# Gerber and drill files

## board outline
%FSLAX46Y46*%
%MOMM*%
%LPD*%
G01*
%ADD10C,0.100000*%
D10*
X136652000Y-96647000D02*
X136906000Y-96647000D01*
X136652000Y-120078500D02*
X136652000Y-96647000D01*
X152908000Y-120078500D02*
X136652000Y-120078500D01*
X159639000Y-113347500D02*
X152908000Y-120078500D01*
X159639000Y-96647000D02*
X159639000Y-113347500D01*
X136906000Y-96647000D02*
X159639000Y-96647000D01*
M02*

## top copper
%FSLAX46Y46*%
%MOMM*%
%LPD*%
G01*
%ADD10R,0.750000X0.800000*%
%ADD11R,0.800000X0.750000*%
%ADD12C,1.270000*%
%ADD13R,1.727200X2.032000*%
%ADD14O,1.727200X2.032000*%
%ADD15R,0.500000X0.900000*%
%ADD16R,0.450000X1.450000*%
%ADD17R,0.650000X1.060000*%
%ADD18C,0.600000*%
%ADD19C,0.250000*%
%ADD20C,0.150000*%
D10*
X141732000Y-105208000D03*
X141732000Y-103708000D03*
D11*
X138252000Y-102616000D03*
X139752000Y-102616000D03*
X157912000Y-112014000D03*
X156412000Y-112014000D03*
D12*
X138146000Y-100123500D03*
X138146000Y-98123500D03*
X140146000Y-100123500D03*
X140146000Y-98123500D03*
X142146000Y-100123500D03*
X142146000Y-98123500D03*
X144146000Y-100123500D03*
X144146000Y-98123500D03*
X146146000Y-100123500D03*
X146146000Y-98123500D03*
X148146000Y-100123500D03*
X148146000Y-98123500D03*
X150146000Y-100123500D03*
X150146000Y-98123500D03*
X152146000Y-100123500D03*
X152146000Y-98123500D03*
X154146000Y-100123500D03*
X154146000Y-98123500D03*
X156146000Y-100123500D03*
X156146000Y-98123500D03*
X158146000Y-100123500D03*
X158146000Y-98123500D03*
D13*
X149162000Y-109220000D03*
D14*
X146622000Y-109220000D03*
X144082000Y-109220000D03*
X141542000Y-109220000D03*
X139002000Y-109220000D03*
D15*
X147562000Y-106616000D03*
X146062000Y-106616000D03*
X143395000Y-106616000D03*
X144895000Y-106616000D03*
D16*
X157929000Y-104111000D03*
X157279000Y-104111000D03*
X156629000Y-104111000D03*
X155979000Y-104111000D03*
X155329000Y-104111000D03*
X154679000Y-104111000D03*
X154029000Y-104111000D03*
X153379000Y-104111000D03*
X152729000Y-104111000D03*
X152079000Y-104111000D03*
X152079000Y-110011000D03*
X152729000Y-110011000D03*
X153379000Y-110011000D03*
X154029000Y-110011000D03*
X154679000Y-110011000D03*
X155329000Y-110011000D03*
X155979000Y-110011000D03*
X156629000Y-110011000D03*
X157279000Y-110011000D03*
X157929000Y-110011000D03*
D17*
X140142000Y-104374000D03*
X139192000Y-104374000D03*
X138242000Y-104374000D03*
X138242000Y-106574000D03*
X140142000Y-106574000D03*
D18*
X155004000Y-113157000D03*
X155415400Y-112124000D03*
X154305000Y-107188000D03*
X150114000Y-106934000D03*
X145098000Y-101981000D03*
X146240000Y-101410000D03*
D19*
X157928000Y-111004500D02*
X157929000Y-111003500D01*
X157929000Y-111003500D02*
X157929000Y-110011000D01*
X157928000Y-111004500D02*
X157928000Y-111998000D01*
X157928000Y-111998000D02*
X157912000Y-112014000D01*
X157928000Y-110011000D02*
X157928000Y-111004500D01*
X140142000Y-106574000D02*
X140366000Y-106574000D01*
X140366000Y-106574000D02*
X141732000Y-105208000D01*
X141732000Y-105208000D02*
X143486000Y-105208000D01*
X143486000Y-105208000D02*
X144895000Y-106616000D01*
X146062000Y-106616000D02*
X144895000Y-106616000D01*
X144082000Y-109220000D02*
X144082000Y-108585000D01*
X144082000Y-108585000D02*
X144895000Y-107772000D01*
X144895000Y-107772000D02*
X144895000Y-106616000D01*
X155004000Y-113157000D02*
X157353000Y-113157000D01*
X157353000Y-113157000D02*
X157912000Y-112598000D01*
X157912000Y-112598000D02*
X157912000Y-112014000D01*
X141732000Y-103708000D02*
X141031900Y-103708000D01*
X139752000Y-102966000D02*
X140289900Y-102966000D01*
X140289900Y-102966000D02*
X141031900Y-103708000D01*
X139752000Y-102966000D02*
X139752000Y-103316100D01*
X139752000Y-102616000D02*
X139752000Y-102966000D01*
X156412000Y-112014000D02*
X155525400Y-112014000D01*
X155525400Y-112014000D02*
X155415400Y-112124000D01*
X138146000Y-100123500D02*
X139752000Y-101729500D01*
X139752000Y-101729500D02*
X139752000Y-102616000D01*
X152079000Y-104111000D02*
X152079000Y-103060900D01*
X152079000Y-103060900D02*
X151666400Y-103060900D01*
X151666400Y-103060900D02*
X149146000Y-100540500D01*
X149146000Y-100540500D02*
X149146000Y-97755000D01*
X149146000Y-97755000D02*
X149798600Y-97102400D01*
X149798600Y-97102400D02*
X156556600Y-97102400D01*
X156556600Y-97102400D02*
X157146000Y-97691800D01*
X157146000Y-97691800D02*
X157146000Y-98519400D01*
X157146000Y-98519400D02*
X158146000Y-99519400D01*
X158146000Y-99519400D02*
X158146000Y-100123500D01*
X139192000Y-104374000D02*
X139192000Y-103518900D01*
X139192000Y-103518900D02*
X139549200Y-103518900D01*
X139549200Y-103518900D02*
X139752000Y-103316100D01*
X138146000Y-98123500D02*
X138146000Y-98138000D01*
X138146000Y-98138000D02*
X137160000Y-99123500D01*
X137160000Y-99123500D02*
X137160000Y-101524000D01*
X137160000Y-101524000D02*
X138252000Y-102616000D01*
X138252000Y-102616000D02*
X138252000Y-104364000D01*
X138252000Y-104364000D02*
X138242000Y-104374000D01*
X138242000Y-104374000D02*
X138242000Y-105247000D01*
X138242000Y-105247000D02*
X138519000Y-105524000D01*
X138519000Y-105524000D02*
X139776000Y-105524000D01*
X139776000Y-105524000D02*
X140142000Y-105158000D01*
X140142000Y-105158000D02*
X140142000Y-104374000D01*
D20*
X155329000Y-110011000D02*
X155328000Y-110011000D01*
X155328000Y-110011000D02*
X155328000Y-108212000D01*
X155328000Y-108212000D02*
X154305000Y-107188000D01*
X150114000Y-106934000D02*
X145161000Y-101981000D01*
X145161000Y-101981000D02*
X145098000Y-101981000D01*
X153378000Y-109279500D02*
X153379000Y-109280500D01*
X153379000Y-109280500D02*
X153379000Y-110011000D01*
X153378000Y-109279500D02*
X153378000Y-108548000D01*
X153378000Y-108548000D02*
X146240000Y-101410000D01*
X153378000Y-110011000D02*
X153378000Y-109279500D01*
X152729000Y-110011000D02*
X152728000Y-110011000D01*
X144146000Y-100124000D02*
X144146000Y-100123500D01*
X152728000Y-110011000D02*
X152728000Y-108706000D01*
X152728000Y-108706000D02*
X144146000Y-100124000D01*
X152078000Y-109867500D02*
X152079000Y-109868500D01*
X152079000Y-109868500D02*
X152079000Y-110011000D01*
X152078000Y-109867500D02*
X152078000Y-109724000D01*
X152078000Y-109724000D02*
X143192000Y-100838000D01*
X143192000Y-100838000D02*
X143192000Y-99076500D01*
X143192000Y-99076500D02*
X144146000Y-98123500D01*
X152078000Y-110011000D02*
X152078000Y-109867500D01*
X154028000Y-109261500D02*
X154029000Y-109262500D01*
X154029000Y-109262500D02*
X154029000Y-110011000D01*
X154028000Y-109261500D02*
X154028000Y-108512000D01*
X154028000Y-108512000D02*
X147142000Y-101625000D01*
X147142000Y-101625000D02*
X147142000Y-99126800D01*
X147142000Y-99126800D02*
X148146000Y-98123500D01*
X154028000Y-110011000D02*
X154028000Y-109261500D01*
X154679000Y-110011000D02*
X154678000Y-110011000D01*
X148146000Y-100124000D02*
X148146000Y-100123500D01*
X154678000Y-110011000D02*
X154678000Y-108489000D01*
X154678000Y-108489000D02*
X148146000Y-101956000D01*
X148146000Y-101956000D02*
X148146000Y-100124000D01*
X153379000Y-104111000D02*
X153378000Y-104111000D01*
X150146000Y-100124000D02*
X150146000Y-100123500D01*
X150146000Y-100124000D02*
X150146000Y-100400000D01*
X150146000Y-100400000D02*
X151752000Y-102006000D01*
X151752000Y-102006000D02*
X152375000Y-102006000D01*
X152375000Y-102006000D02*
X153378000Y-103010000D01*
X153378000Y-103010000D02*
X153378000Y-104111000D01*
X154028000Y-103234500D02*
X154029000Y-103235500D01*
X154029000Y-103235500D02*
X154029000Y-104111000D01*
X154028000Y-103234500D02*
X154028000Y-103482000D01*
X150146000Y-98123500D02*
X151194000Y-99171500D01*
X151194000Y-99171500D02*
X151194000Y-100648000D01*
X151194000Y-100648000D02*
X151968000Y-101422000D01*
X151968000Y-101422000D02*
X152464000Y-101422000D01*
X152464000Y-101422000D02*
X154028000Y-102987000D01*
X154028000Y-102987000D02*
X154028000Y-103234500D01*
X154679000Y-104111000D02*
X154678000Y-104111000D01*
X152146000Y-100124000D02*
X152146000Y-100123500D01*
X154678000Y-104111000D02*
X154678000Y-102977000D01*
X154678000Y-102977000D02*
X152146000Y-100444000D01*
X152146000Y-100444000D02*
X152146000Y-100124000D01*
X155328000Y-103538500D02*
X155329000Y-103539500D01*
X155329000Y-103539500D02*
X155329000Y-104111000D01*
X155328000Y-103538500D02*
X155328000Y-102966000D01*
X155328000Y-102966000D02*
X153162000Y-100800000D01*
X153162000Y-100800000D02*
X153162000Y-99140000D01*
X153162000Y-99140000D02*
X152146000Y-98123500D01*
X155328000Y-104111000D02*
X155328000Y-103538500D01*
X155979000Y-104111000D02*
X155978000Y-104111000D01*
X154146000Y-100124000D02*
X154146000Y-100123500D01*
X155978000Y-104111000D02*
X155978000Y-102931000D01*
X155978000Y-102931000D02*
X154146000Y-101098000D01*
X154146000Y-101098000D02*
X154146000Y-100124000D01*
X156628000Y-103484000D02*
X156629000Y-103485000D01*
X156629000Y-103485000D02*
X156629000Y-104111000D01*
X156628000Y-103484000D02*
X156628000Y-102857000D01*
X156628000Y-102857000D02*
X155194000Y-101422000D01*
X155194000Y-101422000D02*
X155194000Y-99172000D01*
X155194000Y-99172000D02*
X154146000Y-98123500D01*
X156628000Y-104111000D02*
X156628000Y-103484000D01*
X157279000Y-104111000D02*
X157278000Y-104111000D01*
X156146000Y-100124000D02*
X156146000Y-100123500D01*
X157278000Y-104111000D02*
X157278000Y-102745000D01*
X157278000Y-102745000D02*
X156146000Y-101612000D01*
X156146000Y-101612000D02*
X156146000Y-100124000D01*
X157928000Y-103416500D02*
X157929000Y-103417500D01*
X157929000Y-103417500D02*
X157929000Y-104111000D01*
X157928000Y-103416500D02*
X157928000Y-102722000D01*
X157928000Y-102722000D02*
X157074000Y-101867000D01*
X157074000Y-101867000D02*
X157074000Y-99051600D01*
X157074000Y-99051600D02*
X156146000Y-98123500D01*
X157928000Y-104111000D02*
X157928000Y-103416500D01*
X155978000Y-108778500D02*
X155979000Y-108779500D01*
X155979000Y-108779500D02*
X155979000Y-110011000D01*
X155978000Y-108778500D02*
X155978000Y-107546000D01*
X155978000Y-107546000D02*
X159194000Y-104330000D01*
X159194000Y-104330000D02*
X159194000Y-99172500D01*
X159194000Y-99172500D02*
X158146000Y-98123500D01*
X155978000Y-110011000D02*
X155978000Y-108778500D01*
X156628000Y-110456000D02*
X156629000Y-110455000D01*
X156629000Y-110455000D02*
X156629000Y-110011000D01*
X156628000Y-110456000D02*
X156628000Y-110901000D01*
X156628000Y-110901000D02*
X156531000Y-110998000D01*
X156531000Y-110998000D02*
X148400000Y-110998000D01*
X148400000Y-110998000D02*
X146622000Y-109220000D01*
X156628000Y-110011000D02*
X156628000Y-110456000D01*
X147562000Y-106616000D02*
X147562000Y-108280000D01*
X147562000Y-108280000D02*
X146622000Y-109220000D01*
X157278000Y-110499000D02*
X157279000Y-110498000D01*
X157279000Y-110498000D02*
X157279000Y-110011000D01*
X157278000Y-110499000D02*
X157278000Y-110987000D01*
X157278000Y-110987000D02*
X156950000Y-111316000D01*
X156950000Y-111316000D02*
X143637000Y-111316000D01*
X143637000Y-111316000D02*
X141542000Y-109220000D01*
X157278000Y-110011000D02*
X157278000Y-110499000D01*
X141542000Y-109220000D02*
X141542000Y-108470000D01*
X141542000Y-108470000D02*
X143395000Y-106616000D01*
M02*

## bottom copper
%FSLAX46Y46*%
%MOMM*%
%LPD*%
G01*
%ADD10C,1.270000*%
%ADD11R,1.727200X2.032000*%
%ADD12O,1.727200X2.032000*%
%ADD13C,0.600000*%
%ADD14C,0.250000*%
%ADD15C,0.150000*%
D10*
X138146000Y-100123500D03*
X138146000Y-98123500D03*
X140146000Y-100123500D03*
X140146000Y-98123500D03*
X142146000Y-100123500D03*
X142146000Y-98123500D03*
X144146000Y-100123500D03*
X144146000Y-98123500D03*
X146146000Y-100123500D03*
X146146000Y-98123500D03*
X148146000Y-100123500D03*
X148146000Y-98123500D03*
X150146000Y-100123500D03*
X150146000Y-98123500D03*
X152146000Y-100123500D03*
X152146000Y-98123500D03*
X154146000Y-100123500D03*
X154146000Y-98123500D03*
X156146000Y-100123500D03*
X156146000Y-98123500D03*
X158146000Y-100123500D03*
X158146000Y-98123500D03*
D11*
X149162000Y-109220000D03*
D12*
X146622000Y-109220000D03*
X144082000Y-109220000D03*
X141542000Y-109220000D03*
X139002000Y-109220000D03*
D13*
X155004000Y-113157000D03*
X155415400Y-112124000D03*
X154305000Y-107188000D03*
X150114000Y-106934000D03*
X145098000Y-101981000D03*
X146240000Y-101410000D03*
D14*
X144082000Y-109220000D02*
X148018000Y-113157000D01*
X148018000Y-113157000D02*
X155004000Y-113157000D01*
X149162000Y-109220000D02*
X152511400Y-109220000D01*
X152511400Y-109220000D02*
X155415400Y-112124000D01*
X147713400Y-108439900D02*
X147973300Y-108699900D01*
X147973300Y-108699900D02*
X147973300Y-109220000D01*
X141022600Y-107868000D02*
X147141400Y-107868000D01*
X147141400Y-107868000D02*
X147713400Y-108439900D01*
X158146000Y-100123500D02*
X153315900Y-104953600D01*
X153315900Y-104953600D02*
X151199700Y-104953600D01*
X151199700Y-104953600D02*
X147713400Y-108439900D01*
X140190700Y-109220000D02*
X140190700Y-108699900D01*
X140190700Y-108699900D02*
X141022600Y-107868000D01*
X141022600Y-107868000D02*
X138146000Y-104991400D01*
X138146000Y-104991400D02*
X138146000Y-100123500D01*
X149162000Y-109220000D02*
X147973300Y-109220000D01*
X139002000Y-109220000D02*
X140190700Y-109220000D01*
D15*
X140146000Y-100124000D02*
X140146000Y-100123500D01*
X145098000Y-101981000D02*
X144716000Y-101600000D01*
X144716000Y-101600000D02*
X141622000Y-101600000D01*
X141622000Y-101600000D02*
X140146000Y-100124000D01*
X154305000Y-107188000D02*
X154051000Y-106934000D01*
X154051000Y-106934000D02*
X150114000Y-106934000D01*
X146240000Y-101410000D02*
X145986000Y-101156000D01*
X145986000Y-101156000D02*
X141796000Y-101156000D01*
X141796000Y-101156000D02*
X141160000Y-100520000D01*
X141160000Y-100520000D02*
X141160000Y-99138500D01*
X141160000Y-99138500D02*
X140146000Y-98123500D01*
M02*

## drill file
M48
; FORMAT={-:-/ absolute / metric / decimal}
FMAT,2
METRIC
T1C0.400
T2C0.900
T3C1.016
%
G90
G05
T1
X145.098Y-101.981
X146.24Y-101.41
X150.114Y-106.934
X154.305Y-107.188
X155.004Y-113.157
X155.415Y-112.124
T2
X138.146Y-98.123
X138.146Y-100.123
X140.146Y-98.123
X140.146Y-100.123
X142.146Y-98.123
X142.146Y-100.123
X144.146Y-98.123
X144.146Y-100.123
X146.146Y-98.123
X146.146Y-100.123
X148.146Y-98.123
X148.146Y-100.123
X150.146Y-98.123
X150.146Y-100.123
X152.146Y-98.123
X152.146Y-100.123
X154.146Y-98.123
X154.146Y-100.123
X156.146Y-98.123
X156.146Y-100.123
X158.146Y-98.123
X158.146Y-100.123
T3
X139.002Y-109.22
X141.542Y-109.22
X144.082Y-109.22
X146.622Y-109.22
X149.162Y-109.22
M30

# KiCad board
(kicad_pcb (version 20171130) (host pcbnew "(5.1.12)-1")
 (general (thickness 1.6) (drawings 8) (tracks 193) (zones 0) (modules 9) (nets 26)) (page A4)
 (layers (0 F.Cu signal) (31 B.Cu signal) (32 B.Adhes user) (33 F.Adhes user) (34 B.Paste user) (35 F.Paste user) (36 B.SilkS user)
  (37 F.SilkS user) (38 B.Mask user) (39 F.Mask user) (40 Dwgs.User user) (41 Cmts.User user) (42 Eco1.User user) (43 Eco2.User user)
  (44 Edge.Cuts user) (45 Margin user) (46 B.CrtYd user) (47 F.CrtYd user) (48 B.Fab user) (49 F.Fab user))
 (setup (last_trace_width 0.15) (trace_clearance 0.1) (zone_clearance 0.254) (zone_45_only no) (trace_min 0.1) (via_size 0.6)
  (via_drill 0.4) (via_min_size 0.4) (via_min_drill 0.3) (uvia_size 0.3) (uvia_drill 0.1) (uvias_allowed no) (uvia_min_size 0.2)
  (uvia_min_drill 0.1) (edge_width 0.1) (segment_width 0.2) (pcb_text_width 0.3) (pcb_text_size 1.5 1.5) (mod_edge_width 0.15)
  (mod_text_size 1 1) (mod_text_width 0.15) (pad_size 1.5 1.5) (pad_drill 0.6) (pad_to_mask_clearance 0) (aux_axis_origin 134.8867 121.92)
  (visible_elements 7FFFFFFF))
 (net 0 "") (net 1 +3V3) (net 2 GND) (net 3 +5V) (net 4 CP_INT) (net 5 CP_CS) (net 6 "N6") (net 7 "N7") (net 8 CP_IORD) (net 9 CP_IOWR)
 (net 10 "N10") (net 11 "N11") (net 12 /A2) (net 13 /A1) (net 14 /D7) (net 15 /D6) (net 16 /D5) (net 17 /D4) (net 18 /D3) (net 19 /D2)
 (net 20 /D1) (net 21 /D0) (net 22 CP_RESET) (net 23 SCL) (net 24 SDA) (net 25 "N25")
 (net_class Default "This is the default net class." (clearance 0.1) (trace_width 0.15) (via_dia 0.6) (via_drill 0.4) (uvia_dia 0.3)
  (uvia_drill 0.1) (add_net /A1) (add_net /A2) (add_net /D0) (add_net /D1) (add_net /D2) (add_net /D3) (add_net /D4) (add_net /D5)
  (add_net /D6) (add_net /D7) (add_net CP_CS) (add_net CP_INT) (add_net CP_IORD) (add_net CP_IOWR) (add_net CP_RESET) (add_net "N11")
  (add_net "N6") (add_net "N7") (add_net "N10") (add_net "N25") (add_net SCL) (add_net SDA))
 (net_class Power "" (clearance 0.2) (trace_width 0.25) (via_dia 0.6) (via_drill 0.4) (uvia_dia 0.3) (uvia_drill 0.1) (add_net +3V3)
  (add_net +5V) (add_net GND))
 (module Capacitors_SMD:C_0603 (layer F.Cu) (at 141.732 104.458 90)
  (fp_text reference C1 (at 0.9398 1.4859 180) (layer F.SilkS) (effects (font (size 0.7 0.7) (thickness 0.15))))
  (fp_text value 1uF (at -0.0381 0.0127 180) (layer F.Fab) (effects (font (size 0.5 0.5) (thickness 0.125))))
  (pad 1 smd rect (at -0.75 0 90) (size 0.8 0.75) (layers F.Cu F.Paste F.Mask) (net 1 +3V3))
  (pad 2 smd rect (at 0.75 0 90) (size 0.8 0.75) (layers F.Cu F.Paste F.Mask) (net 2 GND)))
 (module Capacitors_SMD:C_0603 (layer F.Cu) (at 139.002 102.616)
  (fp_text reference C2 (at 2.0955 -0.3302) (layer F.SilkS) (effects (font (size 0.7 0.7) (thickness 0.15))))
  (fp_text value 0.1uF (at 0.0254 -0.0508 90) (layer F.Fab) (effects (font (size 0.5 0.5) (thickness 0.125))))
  (pad 1 smd rect (at -0.75 0) (size 0.8 0.75) (layers F.Cu F.Paste F.Mask) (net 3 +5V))
  (pad 2 smd rect (at 0.75 0) (size 0.8 0.75) (layers F.Cu F.Paste F.Mask) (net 2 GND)))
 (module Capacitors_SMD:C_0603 (layer F.Cu) (at 157.162 112.014 180)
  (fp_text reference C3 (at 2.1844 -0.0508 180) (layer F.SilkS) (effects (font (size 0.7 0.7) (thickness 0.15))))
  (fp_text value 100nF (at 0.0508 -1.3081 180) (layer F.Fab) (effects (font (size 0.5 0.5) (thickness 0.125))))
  (pad 1 smd rect (at -0.75 0 180) (size 0.8 0.75) (layers F.Cu F.Paste F.Mask) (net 1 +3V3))
  (pad 2 smd rect (at 0.75 0 180) (size 0.8 0.75) (layers F.Cu F.Paste F.Mask) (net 2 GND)))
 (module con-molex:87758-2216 (layer F.Cu) (at 148.146 99.1235)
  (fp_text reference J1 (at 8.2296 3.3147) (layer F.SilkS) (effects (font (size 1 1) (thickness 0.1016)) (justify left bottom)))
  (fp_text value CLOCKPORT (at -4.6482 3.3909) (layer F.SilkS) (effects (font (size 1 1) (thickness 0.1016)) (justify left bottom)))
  (pad 1 thru_hole circle (at -10 1) (size 1.27 1.27) (drill 0.9) (layers *.Cu *.Mask) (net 2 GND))
  (pad 2 thru_hole circle (at -10 -1) (size 1.27 1.27) (drill 0.9) (layers *.Cu *.Mask) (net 3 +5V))
  (pad 3 thru_hole circle (at -8 1) (size 1.27 1.27) (drill 0.9) (layers *.Cu *.Mask) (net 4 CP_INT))
  (pad 4 thru_hole circle (at -8 -1) (size 1.27 1.27) (drill 0.9) (layers *.Cu *.Mask) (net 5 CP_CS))
  (pad 5 thru_hole circle (at -6 1) (size 1.27 1.27) (drill 0.9) (layers *.Cu *.Mask) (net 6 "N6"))
  (pad 6 thru_hole circle (at -6 -1) (size 1.27 1.27) (drill 0.9) (layers *.Cu *.Mask) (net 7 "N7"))
  (pad 7 thru_hole circle (at -4 1) (size 1.27 1.27) (drill 0.9) (layers *.Cu *.Mask) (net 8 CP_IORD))
  (pad 8 thru_hole circle (at -4 -1) (size 1.27 1.27) (drill 0.9) (layers *.Cu *.Mask) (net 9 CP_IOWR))
  (pad 9 thru_hole circle (at -2 1) (size 1.27 1.27) (drill 0.9) (layers *.Cu *.Mask) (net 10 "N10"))
  (pad 10 thru_hole circle (at -2 -1) (size 1.27 1.27) (drill 0.9) (layers *.Cu *.Mask) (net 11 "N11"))
  (pad 11 thru_hole circle (at 0 1) (size 1.27 1.27) (drill 0.9) (layers *.Cu *.Mask) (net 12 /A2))
  (pad 12 thru_hole circle (at 0 -1) (size 1.27 1.27) (drill 0.9) (layers *.Cu *.Mask) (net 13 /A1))
  (pad 13 thru_hole circle (at 2 1) (size 1.27 1.27) (drill 0.9) (layers *.Cu *.Mask) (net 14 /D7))
  (pad 14 thru_hole circle (at 2 -1) (size 1.27 1.27) (drill 0.9) (layers *.Cu *.Mask) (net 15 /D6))
  (pad 15 thru_hole circle (at 4 1) (size 1.27 1.27) (drill 0.9) (layers *.Cu *.Mask) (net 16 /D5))
  (pad 16 thru_hole circle (at 4 -1) (size 1.27 1.27) (drill 0.9) (layers *.Cu *.Mask) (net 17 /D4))
  (pad 17 thru_hole circle (at 6 1) (size 1.27 1.27) (drill 0.9) (layers *.Cu *.Mask) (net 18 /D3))
  (pad 18 thru_hole circle (at 6 -1) (size 1.27 1.27) (drill 0.9) (layers *.Cu *.Mask) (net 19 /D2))
  (pad 19 thru_hole circle (at 8 1) (size 1.27 1.27) (drill 0.9) (layers *.Cu *.Mask) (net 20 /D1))
  (pad 20 thru_hole circle (at 8 -1) (size 1.27 1.27) (drill 0.9) (layers *.Cu *.Mask) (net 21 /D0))
  (pad 21 thru_hole circle (at 10 1) (size 1.27 1.27) (drill 0.9) (layers *.Cu *.Mask) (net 2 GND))
  (pad 22 thru_hole circle (at 10 -1) (size 1.27 1.27) (drill 0.9) (layers *.Cu *.Mask) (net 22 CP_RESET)))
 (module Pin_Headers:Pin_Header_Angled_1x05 (layer F.Cu) (at 149.162 109.22 270)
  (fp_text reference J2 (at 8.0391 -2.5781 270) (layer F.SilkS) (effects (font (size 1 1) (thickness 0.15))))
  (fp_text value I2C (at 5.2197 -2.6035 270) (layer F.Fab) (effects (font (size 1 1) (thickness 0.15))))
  (pad 1 thru_hole rect (at 0 0 270) (size 2.032 1.7272) (drill 1.016) (layers *.Cu *.Mask F.SilkS) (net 2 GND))
  (pad 2 thru_hole oval (at 0 2.54 270) (size 2.032 1.7272) (drill 1.016) (layers *.Cu *.Mask F.SilkS) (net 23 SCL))
  (pad 3 thru_hole oval (at 0 5.08 270) (size 2.032 1.7272) (drill 1.016) (layers *.Cu *.Mask F.SilkS) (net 1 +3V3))
  (pad 4 thru_hole oval (at 0 7.62 270) (size 2.032 1.7272) (drill 1.016) (layers *.Cu *.Mask F.SilkS) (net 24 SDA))
  (pad 5 thru_hole oval (at 0 10.16 270) (size 2.032 1.7272) (drill 1.016) (layers *.Cu *.Mask F.SilkS) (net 2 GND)))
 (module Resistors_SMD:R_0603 (layer F.Cu) (at 146.812 106.616 180)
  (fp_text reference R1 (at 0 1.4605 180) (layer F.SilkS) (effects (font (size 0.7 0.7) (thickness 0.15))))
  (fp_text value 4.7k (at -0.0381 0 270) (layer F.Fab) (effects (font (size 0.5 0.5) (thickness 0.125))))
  (pad 1 smd rect (at -0.75 0 180) (size 0.5 0.9) (layers F.Cu F.Paste F.Mask) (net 23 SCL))
  (pad 2 smd rect (at 0.75 0 180) (size 0.5 0.9) (layers F.Cu F.Paste F.Mask) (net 1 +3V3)))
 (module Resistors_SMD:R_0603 (layer F.Cu) (at 144.145 106.616)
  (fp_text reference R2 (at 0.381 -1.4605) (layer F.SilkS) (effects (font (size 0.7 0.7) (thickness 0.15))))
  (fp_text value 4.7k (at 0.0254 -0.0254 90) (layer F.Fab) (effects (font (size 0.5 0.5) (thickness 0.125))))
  (pad 1 smd rect (at -0.75 0) (size 0.5 0.9) (layers F.Cu F.Paste F.Mask) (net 24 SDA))
  (pad 2 smd rect (at 0.75 0) (size 0.5 0.9) (layers F.Cu F.Paste F.Mask) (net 1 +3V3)))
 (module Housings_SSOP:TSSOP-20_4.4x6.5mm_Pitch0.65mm (layer F.Cu) (at 155.004 107.061 270)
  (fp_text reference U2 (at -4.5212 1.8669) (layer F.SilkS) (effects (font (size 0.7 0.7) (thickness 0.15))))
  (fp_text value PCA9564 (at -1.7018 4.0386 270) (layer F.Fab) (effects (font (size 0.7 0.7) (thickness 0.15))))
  (pad 1 smd rect (at -2.95 -2.925 270) (size 1.45 0.45) (layers F.Cu F.Paste F.Mask) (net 21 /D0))
  (pad 2 smd rect (at -2.95 -2.275 270) (size 1.45 0.45) (layers F.Cu F.Paste F.Mask) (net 20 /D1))
  (pad 3 smd rect (at -2.95 -1.625 270) (size 1.45 0.45) (layers F.Cu F.Paste F.Mask) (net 19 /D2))
  (pad 4 smd rect (at -2.95 -0.975 270) (size 1.45 0.45) (layers F.Cu F.Paste F.Mask) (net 18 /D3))
  (pad 5 smd rect (at -2.95 -0.325 270) (size 1.45 0.45) (layers F.Cu F.Paste F.Mask) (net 17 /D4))
  (pad 6 smd rect (at -2.95 0.325 270) (size 1.45 0.45) (layers F.Cu F.Paste F.Mask) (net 16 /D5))
  (pad 7 smd rect (at -2.95 0.975 270) (size 1.45 0.45) (layers F.Cu F.Paste F.Mask) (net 15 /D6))
  (pad 8 smd rect (at -2.95 1.625 270) (size 1.45 0.45) (layers F.Cu F.Paste F.Mask) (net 14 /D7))
  (pad 9 smd rect (at -2.95 2.275 270) (size 1.45 0.45) (layers F.Cu F.Paste F.Mask) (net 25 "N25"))
  (pad 10 smd rect (at -2.95 2.925 270) (size 1.45 0.45) (layers F.Cu F.Paste F.Mask) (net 2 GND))
  (pad 11 smd rect (at 2.95 2.925 270) (size 1.45 0.45) (layers F.Cu F.Paste F.Mask) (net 9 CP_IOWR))
  (pad 12 smd rect (at 2.95 2.275 270) (size 1.45 0.45) (layers F.Cu F.Paste F.Mask) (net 8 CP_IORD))
  (pad 13 smd rect (at 2.95 1.625 270) (size 1.45 0.45) (layers F.Cu F.Paste F.Mask) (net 5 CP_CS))
  (pad 14 smd rect (at 2.95 0.975 270) (size 1.45 0.45) (layers F.Cu F.Paste F.Mask) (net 13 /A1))
  (pad 15 smd rect (at 2.95 0.325 270) (size 1.45 0.45) (layers F.Cu F.Paste F.Mask) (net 12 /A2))
  (pad 16 smd rect (at 2.95 -0.325 270) (size 1.45 0.45) (layers F.Cu F.Paste F.Mask) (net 4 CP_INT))
  (pad 17 smd rect (at 2.95 -0.975 270) (size 1.45 0.45) (layers F.Cu F.Paste F.Mask) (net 22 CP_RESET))
  (pad 18 smd rect (at 2.95 -1.625 270) (size 1.45 0.45) (layers F.Cu F.Paste F.Mask) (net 23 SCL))
  (pad 19 smd rect (at 2.95 -2.275 270) (size 1.45 0.45) (layers F.Cu F.Paste F.Mask) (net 24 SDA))
  (pad 20 smd rect (at 2.95 -2.925 270) (size 1.45 0.45) (layers F.Cu F.Paste F.Mask) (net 1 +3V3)))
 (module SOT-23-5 (layer F.Cu) (at 139.192 105.474 270)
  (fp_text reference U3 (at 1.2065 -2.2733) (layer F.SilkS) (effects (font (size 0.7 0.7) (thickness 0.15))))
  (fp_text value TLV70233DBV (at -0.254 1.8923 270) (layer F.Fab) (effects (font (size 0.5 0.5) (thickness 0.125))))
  (pad 1 smd rect (at -1.1 -0.95 270) (size 1.06 0.65) (layers F.Cu F.Paste F.Mask) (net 3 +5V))
  (pad 2 smd rect (at -1.1 0 270) (size 1.06 0.65) (layers F.Cu F.Paste F.Mask) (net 2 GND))
  (pad 3 smd rect (at -1.1 0.95 270) (size 1.06 0.65) (layers F.Cu F.Paste F.Mask) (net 3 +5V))
  (pad 4 smd rect (at 1.1 0.95 270) (size 1.06 0.65) (layers F.Cu F.Paste F.Mask))
  (pad 5 smd rect (at 1.1 -0.95 270) (size 1.06 0.65) (layers F.Cu F.Paste F.Mask) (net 1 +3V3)))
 (gr_line (start 136.652 96.647) (end 136.906 96.647) (angle 90) (layer Edge.Cuts) (width 0.1))
 (gr_line (start 136.652 120.0785) (end 136.652 96.647) (angle 90) (layer Edge.Cuts) (width 0.1))
 (gr_line (start 152.908 120.0785) (end 136.652 120.0785) (angle 90) (layer Edge.Cuts) (width 0.1))
 (gr_line (start 159.639 113.3475) (end 152.908 120.0785) (angle 90) (layer Edge.Cuts) (width 0.1))
 (gr_line (start 159.639 96.647) (end 159.639 113.3475) (angle 90) (layer Edge.Cuts) (width 0.1))
 (gr_line (start 136.906 96.647) (end 159.639 96.647) (angle 90) (layer Edge.Cuts) (width 0.1))
 (segment (start 157.928 111.0045) (end 157.929 111.0035) (width 0.25) (layer F.Cu) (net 1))
 (segment (start 157.929 111.0035) (end 157.929 110.011) (width 0.25) (layer F.Cu) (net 1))
 (segment (start 157.928 111.0045) (end 157.928 111.998) (width 0.25) (layer F.Cu) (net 1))
 (segment (start 157.928 111.998) (end 157.912 112.014) (width 0.25) (layer F.Cu) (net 1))
 (segment (start 157.928 110.011) (end 157.928 111.0045) (width 0.25) (layer F.Cu) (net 1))
 (segment (start 140.142 106.574) (end 140.366 106.574) (width 0.25) (layer F.Cu) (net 1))
 (segment (start 140.366 106.574) (end 141.732 105.208) (width 0.25) (layer F.Cu) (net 1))
 (segment (start 141.732 105.208) (end 143.486 105.208) (width 0.25) (layer F.Cu) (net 1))
 (segment (start 143.486 105.208) (end 144.895 106.616) (width 0.25) (layer F.Cu) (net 1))
 (segment (start 146.062 106.616) (end 144.895 106.616) (width 0.25) (layer F.Cu) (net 1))
 (segment (start 144.082 109.22) (end 144.082 108.585) (width 0.25) (layer F.Cu) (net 1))
 (segment (start 144.082 108.585) (end 144.895 107.772) (width 0.25) (layer F.Cu) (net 1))
 (segment (start 144.895 107.772) (end 144.895 106.616) (width 0.25) (layer F.Cu) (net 1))
 (segment (start 144.082 109.22) (end 148.018 113.157) (width 0.25) (layer B.Cu) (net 1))
 (segment (start 148.018 113.157) (end 155.004 113.157) (width 0.25) (layer B.Cu) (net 1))
 (segment (start 155.004 113.157) (end 157.353 113.157) (width 0.25) (layer F.Cu) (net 1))
 (segment (start 157.353 113.157) (end 157.912 112.598) (width 0.25) (layer F.Cu) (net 1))
 (segment (start 157.912 112.598) (end 157.912 112.014) (width 0.25) (layer F.Cu) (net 1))
 (via (at 155.004 113.157) (size 0.6) (layers F.Cu B.Cu) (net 1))
 (segment (start 141.732 103.708) (end 141.0319 103.708) (width 0.25) (layer F.Cu) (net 2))
 (segment (start 139.752 102.966) (end 140.2899 102.966) (width 0.25) (layer F.Cu) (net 2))
 (segment (start 140.2899 102.966) (end 141.0319 103.708) (width 0.25) (layer F.Cu) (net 2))
 (segment (start 139.752 102.966) (end 139.752 103.3161) (width 0.25) (layer F.Cu) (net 2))
 (segment (start 139.752 102.616) (end 139.752 102.966) (width 0.25) (layer F.Cu) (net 2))
 (segment (start 156.412 112.014) (end 155.5254 112.014) (width 0.25) (layer F.Cu) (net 2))
 (segment (start 155.5254 112.014) (end 155.4154 112.124) (width 0.25) (layer F.Cu) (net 2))
 (segment (start 149.162 109.22) (end 152.5114 109.22) (width 0.25) (layer B.Cu) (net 2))
 (segment (start 152.5114 109.22) (end 155.4154 112.124) (width 0.25) (layer B.Cu) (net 2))
 (segment (start 138.146 100.1235) (end 139.752 101.7295) (width 0.25) (layer F.Cu) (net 2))
 (segment (start 139.752 101.7295) (end 139.752 102.616) (width 0.25) (layer F.Cu) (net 2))
 (segment (start 147.7134 108.4399) (end 147.9733 108.6999) (width 0.25) (layer B.Cu) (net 2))
 (segment (start 147.9733 108.6999) (end 147.9733 109.22) (width 0.25) (layer B.Cu) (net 2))
 (segment (start 141.0226 107.868) (end 147.1414 107.868) (width 0.25) (layer B.Cu) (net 2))
 (segment (start 147.1414 107.868) (end 147.7134 108.4399) (width 0.25) (layer B.Cu) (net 2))
 (segment (start 158.146 100.1235) (end 153.3159 104.9536) (width 0.25) (layer B.Cu) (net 2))
 (segment (start 153.3159 104.9536) (end 151.1997 104.9536) (width 0.25) (layer B.Cu) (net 2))
 (segment (start 151.1997 104.9536) (end 147.7134 108.4399) (width 0.25) (layer B.Cu) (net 2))
 (segment (start 140.1907 109.22) (end 140.1907 108.6999) (width 0.25) (layer B.Cu) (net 2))
 (segment (start 140.1907 108.6999) (end 141.0226 107.868) (width 0.25) (layer B.Cu) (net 2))
 (segment (start 141.0226 107.868) (end 138.146 104.9914) (width 0.25) (layer B.Cu) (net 2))
 (segment (start 138.146 104.9914) (end 138.146 100.1235) (width 0.25) (layer B.Cu) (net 2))
 (segment (start 149.162 109.22) (end 147.9733 109.22) (width 0.25) (layer B.Cu) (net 2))
 (segment (start 139.002 109.22) (end 140.1907 109.22) (width 0.25) (layer B.Cu) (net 2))
 (segment (start 152.079 104.111) (end 152.079 103.0609) (width 0.25) (layer F.Cu) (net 2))
 (segment (start 152.079 103.0609) (end 151.6664 103.0609) (width 0.25) (layer F.Cu) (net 2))
 (segment (start 151.6664 103.0609) (end 149.146 100.5405) (width 0.25) (layer F.Cu) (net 2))
 (segment (start 149.146 100.5405) (end 149.146 97.755) (width 0.25) (layer F.Cu) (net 2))
 (segment (start 149.146 97.755) (end 149.7986 97.1024) (width 0.25) (layer F.Cu) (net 2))
 (segment (start 149.7986 97.1024) (end 156.5566 97.1024) (width 0.25) (layer F.Cu) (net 2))
 (segment (start 156.5566 97.1024) (end 157.146 97.6918) (width 0.25) (layer F.Cu) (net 2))
 (segment (start 157.146 97.6918) (end 157.146 98.5194) (width 0.25) (layer F.Cu) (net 2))
 (segment (start 157.146 98.5194) (end 158.146 99.5194) (width 0.25) (layer F.Cu) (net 2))
 (segment (start 158.146 99.5194) (end 158.146 100.1235) (width 0.25) (layer F.Cu) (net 2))
 (segment (start 139.192 104.374) (end 139.192 103.5189) (width 0.25) (layer F.Cu) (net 2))
 (segment (start 139.192 103.5189) (end 139.5492 103.5189) (width 0.25) (layer F.Cu) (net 2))
 (segment (start 139.5492 103.5189) (end 139.752 103.3161) (width 0.25) (layer F.Cu) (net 2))
 (via (at 155.4154 112.124) (size 0.6) (layers F.Cu B.Cu) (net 2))
 (segment (start 138.146 98.1235) (end 138.146 98.138) (width 0.25) (layer F.Cu) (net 3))
 (segment (start 138.146 98.138) (end 137.16 99.1235) (width 0.25) (layer F.Cu) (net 3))
 (segment (start 137.16 99.1235) (end 137.16 101.524) (width 0.25) (layer F.Cu) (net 3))
 (segment (start 137.16 101.524) (end 138.252 102.616) (width 0.25) (layer F.Cu) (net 3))
 (segment (start 138.252 102.616) (end 138.252 104.364) (width 0.25) (layer F.Cu) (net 3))
 (segment (start 138.252 104.364) (end 138.242 104.374) (width 0.25) (layer F.Cu) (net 3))
 (segment (start 138.242 104.374) (end 138.242 105.247) (width 0.25) (layer F.Cu) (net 3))
 (segment (start 138.242 105.247) (end 138.519 105.524) (width 0.25) (layer F.Cu) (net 3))
 (segment (start 138.519 105.524) (end 139.776 105.524) (width 0.25) (layer F.Cu) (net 3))
 (segment (start 139.776 105.524) (end 140.142 105.158) (width 0.25) (layer F.Cu) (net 3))
 (segment (start 140.142 105.158) (end 140.142 104.374) (width 0.25) (layer F.Cu) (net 3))
 (segment (start 155.329 110.011) (end 155.328 110.011) (width 0.15) (layer F.Cu) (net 4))
 (segment (start 140.146 100.124) (end 140.146 100.1235) (width 0.15) (layer B.Cu) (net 4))
 (segment (start 145.098 101.981) (end 144.716 101.6) (width 0.15) (layer B.Cu) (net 4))
 (segment (start 144.716 101.6) (end 141.622 101.6) (width 0.15) (layer B.Cu) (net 4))
 (segment (start 141.622 101.6) (end 140.146 100.124) (width 0.15) (layer B.Cu) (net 4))
 (segment (start 155.328 110.011) (end 155.328 108.212) (width 0.15) (layer F.Cu) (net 4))
 (segment (start 155.328 108.212) (end 154.305 107.188) (width 0.15) (layer F.Cu) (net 4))
 (segment (start 154.305 107.188) (end 154.051 106.934) (width 0.15) (layer B.Cu) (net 4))
 (segment (start 154.051 106.934) (end 150.114 106.934) (width 0.15) (layer B.Cu) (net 4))
 (segment (start 150.114 106.934) (end 145.161 101.981) (width 0.15) (layer F.Cu) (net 4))
 (segment (start 145.161 101.981) (end 145.098 101.981) (width 0.15) (layer F.Cu) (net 4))
 (via (at 154.305 107.188) (size 0.6) (layers F.Cu B.Cu) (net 4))
 (via (at 150.114 106.934) (size 0.6) (layers F.Cu B.Cu) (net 4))
 (via (at 145.098 101.981) (size 0.6) (layers F.Cu B.Cu) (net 4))
 (segment (start 153.378 109.2795) (end 153.379 109.2805) (width 0.15) (layer F.Cu) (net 5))
 (segment (start 153.379 109.2805) (end 153.379 110.011) (width 0.15) (layer F.Cu) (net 5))
 (segment (start 153.378 109.2795) (end 153.378 108.548) (width 0.15) (layer F.Cu) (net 5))
 (segment (start 153.378 108.548) (end 146.24 101.41) (width 0.15) (layer F.Cu) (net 5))
 (segment (start 153.378 110.011) (end 153.378 109.2795) (width 0.15) (layer F.Cu) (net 5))
 (segment (start 146.24 101.41) (end 145.986 101.156) (width 0.15) (layer B.Cu) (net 5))
 (segment (start 145.986 101.156) (end 141.796 101.156) (width 0.15) (layer B.Cu) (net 5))
 (segment (start 141.796 101.156) (end 141.16 100.52) (width 0.15) (layer B.Cu) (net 5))
 (segment (start 141.16 100.52) (end 141.16 99.1385) (width 0.15) (layer B.Cu) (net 5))
 (segment (start 141.16 99.1385) (end 140.146 98.1235) (width 0.15) (layer B.Cu) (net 5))
 (via (at 146.24 101.41) (size 0.6) (layers F.Cu B.Cu) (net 5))
 (segment (start 152.729 110.011) (end 152.728 110.011) (width 0.15) (layer F.Cu) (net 8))
 (segment (start 144.146 100.124) (end 144.146 100.1235) (width 0.15) (layer F.Cu) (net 8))
 (segment (start 152.728 110.011) (end 152.728 108.706) (width 0.15) (layer F.Cu) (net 8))
 (segment (start 152.728 108.706) (end 144.146 100.124) (width 0.15) (layer F.Cu) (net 8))
 (segment (start 152.078 109.8675) (end 152.079 109.8685) (width 0.15) (layer F.Cu) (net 9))
 (segment (start 152.079 109.8685) (end 152.079 110.011) (width 0.15) (layer F.Cu) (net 9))
 (segment (start 152.078 109.8675) (end 152.078 109.724) (width 0.15) (layer F.Cu) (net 9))
 (segment (start 152.078 109.724) (end 143.192 100.838) (width 0.15) (layer F.Cu) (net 9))
 (segment (start 143.192 100.838) (end 143.192 99.0765) (width 0.15) (layer F.Cu) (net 9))
 (segment (start 143.192 99.0765) (end 144.146 98.1235) (width 0.15) (layer F.Cu) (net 9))
 (segment (start 152.078 110.011) (end 152.078 109.8675) (width 0.15) (layer F.Cu) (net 9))
 (segment (start 154.028 109.2615) (end 154.029 109.2625) (width 0.15) (layer F.Cu) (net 13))
 (segment (start 154.029 109.2625) (end 154.029 110.011) (width 0.15) (layer F.Cu) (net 13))
 (segment (start 154.028 109.2615) (end 154.028 108.512) (width 0.15) (layer F.Cu) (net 13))
 (segment (start 154.028 108.512) (end 147.142 101.625) (width 0.15) (layer F.Cu) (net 13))
 (segment (start 147.142 101.625) (end 147.142 99.1268) (width 0.15) (layer F.Cu) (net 13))
 (segment (start 147.142 99.1268) (end 148.146 98.1235) (width 0.15) (layer F.Cu) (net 13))
 (segment (start 154.028 110.011) (end 154.028 109.2615) (width 0.15) (layer F.Cu) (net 13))
 (segment (start 154.679 110.011) (end 154.678 110.011) (width 0.15) (layer F.Cu) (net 12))
 (segment (start 148.146 100.124) (end 148.146 100.1235) (width 0.15) (layer F.Cu) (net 12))
 (segment (start 154.678 110.011) (end 154.678 108.489) (width 0.15) (layer F.Cu) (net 12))
 (segment (start 154.678 108.489) (end 148.146 101.956) (width 0.15) (layer F.Cu) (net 12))
 (segment (start 148.146 101.956) (end 148.146 100.124) (width 0.15) (layer F.Cu) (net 12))
 (segment (start 153.379 104.111) (end 153.378 104.111) (width 0.15) (layer F.Cu) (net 14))
 (segment (start 150.146 100.124) (end 150.146 100.1235) (width 0.15) (layer F.Cu) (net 14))
 (segment (start 150.146 100.124) (end 150.146 100.4) (width 0.15) (layer F.Cu) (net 14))
 (segment (start 150.146 100.4) (end 151.752 102.006) (width 0.15) (layer F.Cu) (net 14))
 (segment (start 151.752 102.006) (end 152.375 102.006) (width 0.15) (layer F.Cu) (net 14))
 (segment (start 152.375 102.006) (end 153.378 103.01) (width 0.15) (layer F.Cu) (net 14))
 (segment (start 153.378 103.01) (end 153.378 104.111) (width 0.15) (layer F.Cu) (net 14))
 (segment (start 154.028 103.2345) (end 154.029 103.2355) (width 0.15) (layer F.Cu) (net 15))
 (segment (start 154.029 103.2355) (end 154.029 104.111) (width 0.15) (layer F.Cu) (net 15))
 (segment (start 154.028 103.2345) (end 154.028 103.482) (width 0.15) (layer F.Cu) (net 15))
 (segment (start 150.146 98.1235) (end 151.194 99.1715) (width 0.15) (layer F.Cu) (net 15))
 (segment (start 151.194 99.1715) (end 151.194 100.648) (width 0.15) (layer F.Cu) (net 15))
 (segment (start 151.194 100.648) (end 151.968 101.422) (width 0.15) (layer F.Cu) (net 15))
 (segment (start 151.968 101.422) (end 152.464 101.422) (width 0.15) (layer F.Cu) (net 15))
 (segment (start 152.464 101.422) (end 154.028 102.987) (width 0.15) (layer F.Cu) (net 15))
 (segment (start 154.028 102.987) (end 154.028 103.2345) (width 0.15) (layer F.Cu) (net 15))
 (segment (start 154.679 104.111) (end 154.678 104.111) (width 0.15) (layer F.Cu) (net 16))
 (segment (start 152.146 100.124) (end 152.146 100.1235) (width 0.15) (layer F.Cu) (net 16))
 (segment (start 154.678 104.111) (end 154.678 102.977) (width 0.15) (layer F.Cu) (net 16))
 (segment (start 154.678 102.977) (end 152.146 100.444) (width 0.15) (layer F.Cu) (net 16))
 (segment (start 152.146 100.444) (end 152.146 100.124) (width 0.15) (layer F.Cu) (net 16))
 (segment (start 155.328 103.5385) (end 155.329 103.5395) (width 0.15) (layer F.Cu) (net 17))
 (segment (start 155.329 103.5395) (end 155.329 104.111) (width 0.15) (layer F.Cu) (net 17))
 (segment (start 155.328 103.5385) (end 155.328 102.966) (width 0.15) (layer F.Cu) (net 17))
 (segment (start 155.328 102.966) (end 153.162 100.8) (width 0.15) (layer F.Cu) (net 17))
 (segment (start 153.162 100.8) (end 153.162 99.14) (width 0.15) (layer F.Cu) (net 17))
 (segment (start 153.162 99.14) (end 152.146 98.1235) (width 0.15) (layer F.Cu) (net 17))
 (segment (start 155.328 104.111) (end 155.328 103.5385) (width 0.15) (layer F.Cu) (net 17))
 (segment (start 155.979 104.111) (end 155.978 104.111) (width 0.15) (layer F.Cu) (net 18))
 (segment (start 154.146 100.124) (end 154.146 100.1235) (width 0.15) (layer F.Cu) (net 18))
 (segment (start 155.978 104.111) (end 155.978 102.931) (width 0.15) (layer F.Cu) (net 18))
 (segment (start 155.978 102.931) (end 154.146 101.098) (width 0.15) (layer F.Cu) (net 18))
 (segment (start 154.146 101.098) (end 154.146 100.124) (width 0.15) (layer F.Cu) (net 18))
 (segment (start 156.628 103.484) (end 156.629 103.485) (width 0.15) (layer F.Cu) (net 19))
 (segment (start 156.629 103.485) (end 156.629 104.111) (width 0.15) (layer F.Cu) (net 19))
 (segment (start 156.628 103.484) (end 156.628 102.857) (width 0.15) (layer F.Cu) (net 19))
 (segment (start 156.628 102.857) (end 155.194 101.422) (width 0.15) (layer F.Cu) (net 19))
 (segment (start 155.194 101.422) (end 155.194 99.172) (width 0.15) (layer F.Cu) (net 19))
 (segment (start 155.194 99.172) (end 154.146 98.1235) (width 0.15) (layer F.Cu) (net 19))
 (segment (start 156.628 104.111) (end 156.628 103.484) (width 0.15) (layer F.Cu) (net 19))
 (segment (start 157.279 104.111) (end 157.278 104.111) (width 0.15) (layer F.Cu) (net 20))
 (segment (start 156.146 100.124) (end 156.146 100.1235) (width 0.15) (layer F.Cu) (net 20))
 (segment (start 157.278 104.111) (end 157.278 102.745) (width 0.15) (layer F.Cu) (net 20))
 (segment (start 157.278 102.745) (end 156.146 101.612) (width 0.15) (layer F.Cu) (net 20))
 (segment (start 156.146 101.612) (end 156.146 100.124) (width 0.15) (layer F.Cu) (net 20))
 (segment (start 157.928 103.4165) (end 157.929 103.4175) (width 0.15) (layer F.Cu) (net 21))
 (segment (start 157.929 103.4175) (end 157.929 104.111) (width 0.15) (layer F.Cu) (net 21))
 (segment (start 157.928 103.4165) (end 157.928 102.722) (width 0.15) (layer F.Cu) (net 21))
 (segment (start 157.928 102.722) (end 157.074 101.867) (width 0.15) (layer F.Cu) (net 21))
 (segment (start 157.074 101.867) (end 157.074 99.0516) (width 0.15) (layer F.Cu) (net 21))
 (segment (start 157.074 99.0516) (end 156.146 98.1235) (width 0.15) (layer F.Cu) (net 21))
 (segment (start 157.928 104.111) (end 157.928 103.4165) (width 0.15) (layer F.Cu) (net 21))
 (segment (start 155.978 108.7785) (end 155.979 108.7795) (width 0.15) (layer F.Cu) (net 22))
 (segment (start 155.979 108.7795) (end 155.979 110.011) (width 0.15) (layer F.Cu) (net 22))
 (segment (start 155.978 108.7785) (end 155.978 107.546) (width 0.15) (layer F.Cu) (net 22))
 (segment (start 155.978 107.546) (end 159.194 104.33) (width 0.15) (layer F.Cu) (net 22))
 (segment (start 159.194 104.33) (end 159.194 99.1725) (width 0.15) (layer F.Cu) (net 22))
 (segment (start 159.194 99.1725) (end 158.146 98.1235) (width 0.15) (layer F.Cu) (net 22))
 (segment (start 155.978 110.011) (end 155.978 108.7785) (width 0.15) (layer F.Cu) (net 22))
 (segment (start 156.628 110.456) (end 156.629 110.455) (width 0.15) (layer F.Cu) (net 23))
 (segment (start 156.629 110.455) (end 156.629 110.011) (width 0.15) (layer F.Cu) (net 23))
 (segment (start 156.628 110.456) (end 156.628 110.901) (width 0.15) (layer F.Cu) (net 23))
 (segment (start 156.628 110.901) (end 156.531 110.998) (width 0.15) (layer F.Cu) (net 23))
 (segment (start 156.531 110.998) (end 148.4 110.998) (width 0.15) (layer F.Cu) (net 23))
 (segment (start 148.4 110.998) (end 146.622 109.22) (width 0.15) (layer F.Cu) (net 23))
 (segment (start 156.628 110.011) (end 156.628 110.456) (width 0.15) (layer F.Cu) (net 23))
 (segment (start 147.562 106.616) (end 147.562 108.28) (width 0.15) (layer F.Cu) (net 23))
 (segment (start 147.562 108.28) (end 146.622 109.22) (width 0.15) (layer F.Cu) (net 23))
 (segment (start 157.278 110.499) (end 157.279 110.498) (width 0.15) (layer F.Cu) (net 24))
 (segment (start 157.279 110.498) (end 157.279 110.011) (width 0.15) (layer F.Cu) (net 24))
 (segment (start 157.278 110.499) (end 157.278 110.987) (width 0.15) (layer F.Cu) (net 24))
 (segment (start 157.278 110.987) (end 156.95 111.316) (width 0.15) (layer F.Cu) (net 24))
 (segment (start 156.95 111.316) (end 143.637 111.316) (width 0.15) (layer F.Cu) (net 24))
 (segment (start 143.637 111.316) (end 141.542 109.22) (width 0.15) (layer F.Cu) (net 24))
 (segment (start 157.278 110.011) (end 157.278 110.499) (width 0.15) (layer F.Cu) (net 24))
 (segment (start 141.542 109.22) (end 141.542 108.47) (width 0.15) (layer F.Cu) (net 24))
 (segment (start 141.542 108.47) (end 143.395 106.616) (width 0.15) (layer F.Cu) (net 24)))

